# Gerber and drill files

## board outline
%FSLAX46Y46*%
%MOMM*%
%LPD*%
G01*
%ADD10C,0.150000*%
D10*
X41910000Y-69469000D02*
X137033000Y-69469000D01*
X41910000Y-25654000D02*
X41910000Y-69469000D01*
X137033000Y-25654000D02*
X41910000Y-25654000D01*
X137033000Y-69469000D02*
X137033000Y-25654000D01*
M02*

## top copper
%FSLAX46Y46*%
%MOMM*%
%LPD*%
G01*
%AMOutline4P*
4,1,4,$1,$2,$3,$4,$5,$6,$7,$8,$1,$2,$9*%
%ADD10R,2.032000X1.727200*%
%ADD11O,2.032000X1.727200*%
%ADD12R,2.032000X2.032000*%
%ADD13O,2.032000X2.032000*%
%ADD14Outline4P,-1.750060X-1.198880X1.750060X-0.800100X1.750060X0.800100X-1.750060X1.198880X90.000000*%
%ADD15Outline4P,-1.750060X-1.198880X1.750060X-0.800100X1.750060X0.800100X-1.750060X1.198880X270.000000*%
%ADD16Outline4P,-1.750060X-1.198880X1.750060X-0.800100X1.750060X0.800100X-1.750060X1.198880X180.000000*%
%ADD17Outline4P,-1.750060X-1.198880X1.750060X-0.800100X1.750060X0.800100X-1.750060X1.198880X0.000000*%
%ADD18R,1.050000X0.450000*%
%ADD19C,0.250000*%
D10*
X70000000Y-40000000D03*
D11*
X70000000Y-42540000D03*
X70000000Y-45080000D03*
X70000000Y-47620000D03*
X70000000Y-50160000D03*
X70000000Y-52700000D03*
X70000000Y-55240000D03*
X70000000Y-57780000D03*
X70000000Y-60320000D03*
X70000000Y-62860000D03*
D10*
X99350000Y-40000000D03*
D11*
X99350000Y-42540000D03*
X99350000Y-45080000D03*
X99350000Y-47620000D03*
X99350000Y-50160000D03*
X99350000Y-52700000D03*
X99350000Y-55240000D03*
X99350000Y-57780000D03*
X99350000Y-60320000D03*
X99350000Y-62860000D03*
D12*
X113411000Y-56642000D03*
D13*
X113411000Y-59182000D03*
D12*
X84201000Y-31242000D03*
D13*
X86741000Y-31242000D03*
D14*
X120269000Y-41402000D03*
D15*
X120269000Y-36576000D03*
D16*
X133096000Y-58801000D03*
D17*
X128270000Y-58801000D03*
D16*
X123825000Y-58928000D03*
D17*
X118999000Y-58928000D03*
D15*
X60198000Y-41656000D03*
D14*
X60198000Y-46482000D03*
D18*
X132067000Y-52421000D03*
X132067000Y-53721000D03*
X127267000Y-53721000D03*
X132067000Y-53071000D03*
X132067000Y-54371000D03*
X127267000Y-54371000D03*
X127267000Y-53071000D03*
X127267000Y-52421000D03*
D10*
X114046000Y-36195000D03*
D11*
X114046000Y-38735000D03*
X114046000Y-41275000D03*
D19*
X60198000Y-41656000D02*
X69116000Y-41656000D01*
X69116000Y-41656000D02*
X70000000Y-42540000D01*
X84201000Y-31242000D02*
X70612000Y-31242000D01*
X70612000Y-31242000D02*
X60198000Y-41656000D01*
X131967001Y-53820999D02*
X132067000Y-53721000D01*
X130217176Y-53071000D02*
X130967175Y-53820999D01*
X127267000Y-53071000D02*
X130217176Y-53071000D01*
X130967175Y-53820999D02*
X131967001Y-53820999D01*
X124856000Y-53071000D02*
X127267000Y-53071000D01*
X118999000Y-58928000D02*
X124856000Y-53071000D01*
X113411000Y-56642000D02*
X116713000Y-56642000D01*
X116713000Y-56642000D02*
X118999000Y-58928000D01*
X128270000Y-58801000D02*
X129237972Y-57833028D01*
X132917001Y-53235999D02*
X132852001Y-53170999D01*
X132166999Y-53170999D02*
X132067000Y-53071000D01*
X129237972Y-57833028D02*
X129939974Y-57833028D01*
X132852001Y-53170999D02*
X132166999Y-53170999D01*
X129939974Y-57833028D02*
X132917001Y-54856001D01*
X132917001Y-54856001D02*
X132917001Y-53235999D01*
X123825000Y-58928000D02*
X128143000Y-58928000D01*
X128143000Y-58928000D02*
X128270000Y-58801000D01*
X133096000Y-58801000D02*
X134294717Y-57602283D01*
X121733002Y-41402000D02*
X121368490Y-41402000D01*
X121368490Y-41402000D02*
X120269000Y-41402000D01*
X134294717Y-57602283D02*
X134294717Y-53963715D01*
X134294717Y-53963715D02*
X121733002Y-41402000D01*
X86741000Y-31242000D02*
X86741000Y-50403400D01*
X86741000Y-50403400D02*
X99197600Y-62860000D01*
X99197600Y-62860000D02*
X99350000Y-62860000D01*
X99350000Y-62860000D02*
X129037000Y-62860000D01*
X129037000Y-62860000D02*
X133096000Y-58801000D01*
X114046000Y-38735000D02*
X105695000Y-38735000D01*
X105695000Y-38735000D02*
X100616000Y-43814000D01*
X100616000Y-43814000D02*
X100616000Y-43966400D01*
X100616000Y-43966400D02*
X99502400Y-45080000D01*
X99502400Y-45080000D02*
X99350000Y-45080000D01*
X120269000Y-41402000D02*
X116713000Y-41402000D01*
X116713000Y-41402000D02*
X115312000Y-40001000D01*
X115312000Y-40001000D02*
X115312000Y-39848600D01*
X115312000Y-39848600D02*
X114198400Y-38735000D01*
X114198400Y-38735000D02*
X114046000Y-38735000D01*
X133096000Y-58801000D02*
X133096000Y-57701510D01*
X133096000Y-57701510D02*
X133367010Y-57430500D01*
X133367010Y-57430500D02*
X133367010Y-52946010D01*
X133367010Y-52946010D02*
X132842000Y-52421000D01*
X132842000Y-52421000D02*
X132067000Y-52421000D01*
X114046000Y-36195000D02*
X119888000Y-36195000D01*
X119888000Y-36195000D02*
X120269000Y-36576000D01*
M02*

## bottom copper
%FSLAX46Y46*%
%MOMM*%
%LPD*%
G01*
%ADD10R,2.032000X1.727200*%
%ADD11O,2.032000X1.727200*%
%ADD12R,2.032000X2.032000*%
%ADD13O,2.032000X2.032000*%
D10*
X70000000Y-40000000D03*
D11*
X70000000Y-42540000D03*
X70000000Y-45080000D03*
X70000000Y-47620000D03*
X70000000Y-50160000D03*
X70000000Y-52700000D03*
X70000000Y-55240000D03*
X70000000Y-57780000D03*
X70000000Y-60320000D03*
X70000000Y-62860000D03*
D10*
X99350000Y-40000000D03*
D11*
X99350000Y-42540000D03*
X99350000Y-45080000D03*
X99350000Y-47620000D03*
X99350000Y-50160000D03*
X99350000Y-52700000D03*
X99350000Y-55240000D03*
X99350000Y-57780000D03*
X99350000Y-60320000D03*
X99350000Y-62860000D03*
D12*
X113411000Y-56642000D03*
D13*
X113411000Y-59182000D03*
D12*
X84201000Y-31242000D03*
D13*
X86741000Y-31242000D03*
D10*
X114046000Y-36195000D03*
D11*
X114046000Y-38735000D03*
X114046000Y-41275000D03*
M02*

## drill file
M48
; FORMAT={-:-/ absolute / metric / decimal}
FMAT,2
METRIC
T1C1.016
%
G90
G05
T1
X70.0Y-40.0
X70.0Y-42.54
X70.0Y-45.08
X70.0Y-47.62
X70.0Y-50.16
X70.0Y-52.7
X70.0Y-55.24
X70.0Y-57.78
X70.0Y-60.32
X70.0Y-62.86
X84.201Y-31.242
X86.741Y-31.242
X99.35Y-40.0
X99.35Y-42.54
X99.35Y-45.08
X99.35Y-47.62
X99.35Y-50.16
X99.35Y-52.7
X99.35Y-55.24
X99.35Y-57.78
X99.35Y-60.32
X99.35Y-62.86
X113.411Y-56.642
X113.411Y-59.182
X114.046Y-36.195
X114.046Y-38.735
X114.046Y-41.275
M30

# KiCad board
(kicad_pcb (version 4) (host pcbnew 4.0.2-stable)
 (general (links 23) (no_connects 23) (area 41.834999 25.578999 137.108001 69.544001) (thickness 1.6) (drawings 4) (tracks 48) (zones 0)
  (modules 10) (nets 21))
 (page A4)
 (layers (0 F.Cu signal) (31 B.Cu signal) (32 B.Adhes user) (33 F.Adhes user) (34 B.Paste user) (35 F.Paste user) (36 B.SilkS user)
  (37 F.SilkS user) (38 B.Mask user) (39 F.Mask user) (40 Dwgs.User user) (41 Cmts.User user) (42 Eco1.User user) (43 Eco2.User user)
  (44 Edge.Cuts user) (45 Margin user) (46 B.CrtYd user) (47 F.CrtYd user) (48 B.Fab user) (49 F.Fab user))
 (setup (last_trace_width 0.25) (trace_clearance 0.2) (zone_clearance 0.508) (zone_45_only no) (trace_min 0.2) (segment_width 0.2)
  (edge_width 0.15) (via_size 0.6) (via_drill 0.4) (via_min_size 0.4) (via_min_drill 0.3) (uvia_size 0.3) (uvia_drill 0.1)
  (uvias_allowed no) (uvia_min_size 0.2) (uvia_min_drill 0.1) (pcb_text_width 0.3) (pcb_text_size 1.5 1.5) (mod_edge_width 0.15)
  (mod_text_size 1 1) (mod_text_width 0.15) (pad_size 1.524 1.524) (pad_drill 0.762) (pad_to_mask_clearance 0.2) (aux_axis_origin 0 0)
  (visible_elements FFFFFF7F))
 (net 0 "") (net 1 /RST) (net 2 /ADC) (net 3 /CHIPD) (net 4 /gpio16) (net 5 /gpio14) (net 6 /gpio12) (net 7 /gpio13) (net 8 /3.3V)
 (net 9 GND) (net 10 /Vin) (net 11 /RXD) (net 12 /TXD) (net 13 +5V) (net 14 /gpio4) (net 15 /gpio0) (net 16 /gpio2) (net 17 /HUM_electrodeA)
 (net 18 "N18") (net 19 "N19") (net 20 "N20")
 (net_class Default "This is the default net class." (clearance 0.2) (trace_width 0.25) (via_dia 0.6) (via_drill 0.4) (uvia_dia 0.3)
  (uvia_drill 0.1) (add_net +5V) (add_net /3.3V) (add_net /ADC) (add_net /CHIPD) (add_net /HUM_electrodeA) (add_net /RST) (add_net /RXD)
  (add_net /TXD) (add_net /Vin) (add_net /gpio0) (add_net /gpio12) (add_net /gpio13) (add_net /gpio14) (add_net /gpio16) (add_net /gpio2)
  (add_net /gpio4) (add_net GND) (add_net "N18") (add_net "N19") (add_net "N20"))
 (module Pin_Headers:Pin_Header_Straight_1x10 (layer F.Cu) (at 70 40)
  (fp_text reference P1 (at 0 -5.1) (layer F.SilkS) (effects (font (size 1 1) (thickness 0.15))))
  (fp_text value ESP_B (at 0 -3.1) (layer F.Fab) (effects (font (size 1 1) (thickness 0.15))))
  (pad 1 thru_hole rect (at 0 0) (size 2.032 1.7272) (drill 1.016) (layers *.Cu *.Mask F.SilkS) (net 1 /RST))
  (pad 2 thru_hole oval (at 0 2.54) (size 2.032 1.7272) (drill 1.016) (layers *.Cu *.Mask F.SilkS) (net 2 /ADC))
  (pad 3 thru_hole oval (at 0 5.08) (size 2.032 1.7272) (drill 1.016) (layers *.Cu *.Mask F.SilkS) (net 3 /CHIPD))
  (pad 4 thru_hole oval (at 0 7.62) (size 2.032 1.7272) (drill 1.016) (layers *.Cu *.Mask F.SilkS) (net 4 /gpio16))
  (pad 5 thru_hole oval (at 0 10.16) (size 2.032 1.7272) (drill 1.016) (layers *.Cu *.Mask F.SilkS) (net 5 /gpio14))
  (pad 6 thru_hole oval (at 0 12.7) (size 2.032 1.7272) (drill 1.016) (layers *.Cu *.Mask F.SilkS) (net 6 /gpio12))
  (pad 7 thru_hole oval (at 0 15.24) (size 2.032 1.7272) (drill 1.016) (layers *.Cu *.Mask F.SilkS) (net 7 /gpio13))
  (pad 8 thru_hole oval (at 0 17.78) (size 2.032 1.7272) (drill 1.016) (layers *.Cu *.Mask F.SilkS) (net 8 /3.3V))
  (pad 9 thru_hole oval (at 0 20.32) (size 2.032 1.7272) (drill 1.016) (layers *.Cu *.Mask F.SilkS) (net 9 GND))
  (pad 10 thru_hole oval (at 0 22.86) (size 2.032 1.7272) (drill 1.016) (layers *.Cu *.Mask F.SilkS) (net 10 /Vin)))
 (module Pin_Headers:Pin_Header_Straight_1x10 (layer F.Cu) (at 99.35 40)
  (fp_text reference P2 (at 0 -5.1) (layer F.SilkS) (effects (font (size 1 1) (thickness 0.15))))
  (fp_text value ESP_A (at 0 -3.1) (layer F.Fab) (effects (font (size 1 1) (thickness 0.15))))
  (pad 1 thru_hole rect (at 0 0) (size 2.032 1.7272) (drill 1.016) (layers *.Cu *.Mask F.SilkS) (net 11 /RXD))
  (pad 2 thru_hole oval (at 0 2.54) (size 2.032 1.7272) (drill 1.016) (layers *.Cu *.Mask F.SilkS) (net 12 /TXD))
  (pad 3 thru_hole oval (at 0 5.08) (size 2.032 1.7272) (drill 1.016) (layers *.Cu *.Mask F.SilkS) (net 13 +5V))
  (pad 4 thru_hole oval (at 0 7.62) (size 2.032 1.7272) (drill 1.016) (layers *.Cu *.Mask F.SilkS) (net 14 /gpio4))
  (pad 5 thru_hole oval (at 0 10.16) (size 2.032 1.7272) (drill 1.016) (layers *.Cu *.Mask F.SilkS) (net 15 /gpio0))
  (pad 6 thru_hole oval (at 0 12.7) (size 2.032 1.7272) (drill 1.016) (layers *.Cu *.Mask F.SilkS) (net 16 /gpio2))
  (pad 7 thru_hole oval (at 0 15.24) (size 2.032 1.7272) (drill 1.016) (layers *.Cu *.Mask F.SilkS) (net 7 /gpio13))
  (pad 8 thru_hole oval (at 0 17.78) (size 2.032 1.7272) (drill 1.016) (layers *.Cu *.Mask F.SilkS) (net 8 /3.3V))
  (pad 9 thru_hole oval (at 0 20.32) (size 2.032 1.7272) (drill 1.016) (layers *.Cu *.Mask F.SilkS) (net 9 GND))
  (pad 10 thru_hole oval (at 0 22.86) (size 2.032 1.7272) (drill 1.016) (layers *.Cu *.Mask F.SilkS) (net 13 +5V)))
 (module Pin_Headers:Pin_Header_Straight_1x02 (layer F.Cu) (at 113.411 56.642)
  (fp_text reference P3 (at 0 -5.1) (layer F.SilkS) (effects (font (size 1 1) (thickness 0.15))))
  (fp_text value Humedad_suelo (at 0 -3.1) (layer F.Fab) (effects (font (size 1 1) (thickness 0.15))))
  (pad 1 thru_hole rect (at 0 0) (size 2.032 2.032) (drill 1.016) (layers *.Cu *.Mask F.SilkS) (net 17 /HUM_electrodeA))
  (pad 2 thru_hole oval (at 0 2.54) (size 2.032 2.032) (drill 1.016) (layers *.Cu *.Mask F.SilkS) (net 9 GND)))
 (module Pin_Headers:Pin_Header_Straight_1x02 (layer F.Cu) (at 84.201 31.242 90)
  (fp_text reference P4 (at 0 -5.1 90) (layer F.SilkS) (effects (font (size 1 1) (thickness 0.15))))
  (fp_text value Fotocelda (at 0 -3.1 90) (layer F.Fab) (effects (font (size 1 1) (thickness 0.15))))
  (pad 1 thru_hole rect (at 0 0 90) (size 2.032 2.032) (drill 1.016) (layers *.Cu *.Mask F.SilkS) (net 2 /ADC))
  (pad 2 thru_hole oval (at 0 2.54 90) (size 2.032 2.032) (drill 1.016) (layers *.Cu *.Mask F.SilkS) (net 13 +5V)))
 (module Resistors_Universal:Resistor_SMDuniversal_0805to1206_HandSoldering (layer F.Cu) (at 120.269 38.989 90)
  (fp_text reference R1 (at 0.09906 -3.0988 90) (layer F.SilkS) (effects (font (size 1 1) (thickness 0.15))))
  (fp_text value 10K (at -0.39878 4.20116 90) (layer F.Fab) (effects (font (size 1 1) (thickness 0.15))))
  (pad 1 smd trapezoid (at -2.413 0 90) (size 3.50012 1.99898) (rect_delta 0.39878 0) (layers F.Cu F.Paste F.Mask) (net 13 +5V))
  (pad 2 smd trapezoid (at 2.413 0 270) (size 3.50012 1.99898) (rect_delta 0.39878 0) (layers F.Cu F.Paste F.Mask) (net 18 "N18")))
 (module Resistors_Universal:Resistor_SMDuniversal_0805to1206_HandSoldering (layer F.Cu) (at 130.683 58.801 180)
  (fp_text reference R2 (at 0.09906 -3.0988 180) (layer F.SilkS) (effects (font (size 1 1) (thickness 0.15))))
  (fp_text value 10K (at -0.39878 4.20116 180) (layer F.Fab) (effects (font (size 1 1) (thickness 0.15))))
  (pad 1 smd trapezoid (at -2.413 0 180) (size 3.50012 1.99898) (rect_delta 0.39878 0) (layers F.Cu F.Paste F.Mask) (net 13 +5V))
  (pad 2 smd trapezoid (at 2.413 0) (size 3.50012 1.99898) (rect_delta 0.39878 0) (layers F.Cu F.Paste F.Mask) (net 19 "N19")))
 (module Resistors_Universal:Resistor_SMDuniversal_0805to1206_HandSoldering (layer F.Cu) (at 121.412 58.928 180)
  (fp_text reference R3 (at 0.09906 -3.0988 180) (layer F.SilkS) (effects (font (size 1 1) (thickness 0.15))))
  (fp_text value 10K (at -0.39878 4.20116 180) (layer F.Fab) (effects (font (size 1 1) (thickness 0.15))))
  (pad 1 smd trapezoid (at -2.413 0 180) (size 3.50012 1.99898) (rect_delta 0.39878 0) (layers F.Cu F.Paste F.Mask) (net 19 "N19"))
  (pad 2 smd trapezoid (at 2.413 0) (size 3.50012 1.99898) (rect_delta 0.39878 0) (layers F.Cu F.Paste F.Mask) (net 17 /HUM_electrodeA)))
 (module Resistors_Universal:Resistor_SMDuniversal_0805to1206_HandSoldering (layer F.Cu) (at 60.198 44.069 270)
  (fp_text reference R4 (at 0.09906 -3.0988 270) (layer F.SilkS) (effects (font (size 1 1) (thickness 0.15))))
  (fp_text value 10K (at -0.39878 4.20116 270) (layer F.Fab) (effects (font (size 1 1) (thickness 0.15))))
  (pad 1 smd trapezoid (at -2.413 0 270) (size 3.50012 1.99898) (rect_delta 0.39878 0) (layers F.Cu F.Paste F.Mask) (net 2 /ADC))
  (pad 2 smd trapezoid (at 2.413 0 90) (size 3.50012 1.99898) (rect_delta 0.39878 0) (layers F.Cu F.Paste F.Mask) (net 9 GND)))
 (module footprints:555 (layer F.Cu) (at 129.667 53.721 270)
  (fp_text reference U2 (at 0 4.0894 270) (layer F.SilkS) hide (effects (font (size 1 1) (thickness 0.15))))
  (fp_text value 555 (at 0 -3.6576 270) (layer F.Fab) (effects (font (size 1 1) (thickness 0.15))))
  (pad 8 smd rect (at -1.3 -2.4 270) (size 0.45 1.05) (layers F.Cu F.Paste F.Mask) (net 13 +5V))
  (pad 6 smd rect (at 0 -2.4 270) (size 0.45 1.05) (layers F.Cu F.Paste F.Mask) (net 17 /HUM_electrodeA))
  (pad 3 smd rect (at 0 2.4 270) (size 0.45 1.05) (layers F.Cu F.Paste F.Mask) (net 14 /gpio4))
  (pad 7 smd rect (at -0.65 -2.4 270) (size 0.45 1.05) (layers F.Cu F.Paste F.Mask) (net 19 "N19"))
  (pad 5 smd rect (at 0.65 -2.4 270) (size 0.45 1.05) (layers F.Cu F.Paste F.Mask) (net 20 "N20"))
  (pad 4 smd rect (at 0.65 2.4 270) (size 0.45 1.05) (layers F.Cu F.Paste F.Mask) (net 13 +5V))
  (pad 2 smd rect (at -0.65 2.4 270) (size 0.45 1.05) (layers F.Cu F.Paste F.Mask) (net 17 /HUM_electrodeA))
  (pad 1 smd rect (at -1.3 2.4 270) (size 0.45 1.05) (layers F.Cu F.Paste F.Mask) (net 9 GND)))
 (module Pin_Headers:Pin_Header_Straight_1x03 (layer F.Cu) (at 114.046 36.195)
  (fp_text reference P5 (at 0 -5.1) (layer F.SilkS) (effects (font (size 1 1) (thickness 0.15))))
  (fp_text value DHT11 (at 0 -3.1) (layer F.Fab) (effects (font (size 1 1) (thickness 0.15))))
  (pad 1 thru_hole rect (at 0 0) (size 2.032 1.7272) (drill 1.016) (layers *.Cu *.Mask F.SilkS) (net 18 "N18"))
  (pad 2 thru_hole oval (at 0 2.54) (size 2.032 1.7272) (drill 1.016) (layers *.Cu *.Mask F.SilkS) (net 13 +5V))
  (pad 3 thru_hole oval (at 0 5.08) (size 2.032 1.7272) (drill 1.016) (layers *.Cu *.Mask F.SilkS) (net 9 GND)))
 (gr_line (start 41.91 69.469) (end 137.033 69.469) (angle 90) (layer Edge.Cuts) (width 0.15))
 (gr_line (start 41.91 25.654) (end 41.91 69.469) (angle 90) (layer Edge.Cuts) (width 0.15))
 (gr_line (start 137.033 25.654) (end 41.91 25.654) (angle 90) (layer Edge.Cuts) (width 0.15))
 (gr_line (start 137.033 69.469) (end 137.033 25.654) (angle 90) (layer Edge.Cuts) (width 0.15))
 (segment (start 60.198 41.656) (end 69.116 41.656) (width 0.25) (layer F.Cu) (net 2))
 (segment (start 69.116 41.656) (end 70 42.54) (width 0.25) (layer F.Cu) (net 2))
 (segment (start 84.201 31.242) (end 70.612 31.242) (width 0.25) (layer F.Cu) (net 2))
 (segment (start 70.612 31.242) (end 60.198 41.656) (width 0.25) (layer F.Cu) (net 2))
 (segment (start 131.967001 53.820999) (end 132.067 53.721) (width 0.25) (layer F.Cu) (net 17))
 (segment (start 130.217176 53.071) (end 130.967175 53.820999) (width 0.25) (layer F.Cu) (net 17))
 (segment (start 127.267 53.071) (end 130.217176 53.071) (width 0.25) (layer F.Cu) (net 17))
 (segment (start 130.967175 53.820999) (end 131.967001 53.820999) (width 0.25) (layer F.Cu) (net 17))
 (segment (start 124.856 53.071) (end 127.267 53.071) (width 0.25) (layer F.Cu) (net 17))
 (segment (start 118.999 58.928) (end 124.856 53.071) (width 0.25) (layer F.Cu) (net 17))
 (segment (start 113.411 56.642) (end 116.713 56.642) (width 0.25) (layer F.Cu) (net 17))
 (segment (start 116.713 56.642) (end 118.999 58.928) (width 0.25) (layer F.Cu) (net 17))
 (segment (start 128.27 58.801) (end 129.237972 57.833028) (width 0.25) (layer F.Cu) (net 19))
 (segment (start 132.917001 53.235999) (end 132.852001 53.170999) (width 0.25) (layer F.Cu) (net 19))
 (segment (start 132.166999 53.170999) (end 132.067 53.071) (width 0.25) (layer F.Cu) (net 19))
 (segment (start 129.237972 57.833028) (end 129.939974 57.833028) (width 0.25) (layer F.Cu) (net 19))
 (segment (start 132.852001 53.170999) (end 132.166999 53.170999) (width 0.25) (layer F.Cu) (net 19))
 (segment (start 129.939974 57.833028) (end 132.917001 54.856001) (width 0.25) (layer F.Cu) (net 19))
 (segment (start 132.917001 54.856001) (end 132.917001 53.235999) (width 0.25) (layer F.Cu) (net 19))
 (segment (start 123.825 58.928) (end 128.143 58.928) (width 0.25) (layer F.Cu) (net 19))
 (segment (start 128.143 58.928) (end 128.27 58.801) (width 0.25) (layer F.Cu) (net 19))
 (segment (start 133.096 58.801) (end 134.294717 57.602283) (width 0.25) (layer F.Cu) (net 13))
 (segment (start 121.733002 41.402) (end 121.36849 41.402) (width 0.25) (layer F.Cu) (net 13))
 (segment (start 121.36849 41.402) (end 120.269 41.402) (width 0.25) (layer F.Cu) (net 13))
 (segment (start 134.294717 57.602283) (end 134.294717 53.963715) (width 0.25) (layer F.Cu) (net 13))
 (segment (start 134.294717 53.963715) (end 121.733002 41.402) (width 0.25) (layer F.Cu) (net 13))
 (segment (start 86.741 31.242) (end 86.741 50.4034) (width 0.25) (layer F.Cu) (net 13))
 (segment (start 86.741 50.4034) (end 99.1976 62.86) (width 0.25) (layer F.Cu) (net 13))
 (segment (start 99.1976 62.86) (end 99.35 62.86) (width 0.25) (layer F.Cu) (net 13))
 (segment (start 99.35 62.86) (end 129.037 62.86) (width 0.25) (layer F.Cu) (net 13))
 (segment (start 129.037 62.86) (end 133.096 58.801) (width 0.25) (layer F.Cu) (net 13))
 (segment (start 114.046 38.735) (end 105.695 38.735) (width 0.25) (layer F.Cu) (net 13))
 (segment (start 105.695 38.735) (end 100.616 43.814) (width 0.25) (layer F.Cu) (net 13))
 (segment (start 100.616 43.814) (end 100.616 43.9664) (width 0.25) (layer F.Cu) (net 13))
 (segment (start 100.616 43.9664) (end 99.5024 45.08) (width 0.25) (layer F.Cu) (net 13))
 (segment (start 99.5024 45.08) (end 99.35 45.08) (width 0.25) (layer F.Cu) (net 13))
 (segment (start 120.269 41.402) (end 116.713 41.402) (width 0.25) (layer F.Cu) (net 13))
 (segment (start 116.713 41.402) (end 115.312 40.001) (width 0.25) (layer F.Cu) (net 13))
 (segment (start 115.312 40.001) (end 115.312 39.8486) (width 0.25) (layer F.Cu) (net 13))
 (segment (start 115.312 39.8486) (end 114.1984 38.735) (width 0.25) (layer F.Cu) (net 13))
 (segment (start 114.1984 38.735) (end 114.046 38.735) (width 0.25) (layer F.Cu) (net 13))
 (segment (start 133.096 58.801) (end 133.096 57.70151) (width 0.25) (layer F.Cu) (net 13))
 (segment (start 133.096 57.70151) (end 133.36701 57.4305) (width 0.25) (layer F.Cu) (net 13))
 (segment (start 133.36701 57.4305) (end 133.36701 52.94601) (width 0.25) (layer F.Cu) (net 13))
 (segment (start 133.36701 52.94601) (end 132.842 52.421) (width 0.25) (layer F.Cu) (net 13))
 (segment (start 132.842 52.421) (end 132.067 52.421) (width 0.25) (layer F.Cu) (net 13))
 (segment (start 114.046 36.195) (end 119.888 36.195) (width 0.25) (layer F.Cu) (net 18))
 (segment (start 119.888 36.195) (end 120.269 36.576) (width 0.25) (layer F.Cu) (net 18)))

